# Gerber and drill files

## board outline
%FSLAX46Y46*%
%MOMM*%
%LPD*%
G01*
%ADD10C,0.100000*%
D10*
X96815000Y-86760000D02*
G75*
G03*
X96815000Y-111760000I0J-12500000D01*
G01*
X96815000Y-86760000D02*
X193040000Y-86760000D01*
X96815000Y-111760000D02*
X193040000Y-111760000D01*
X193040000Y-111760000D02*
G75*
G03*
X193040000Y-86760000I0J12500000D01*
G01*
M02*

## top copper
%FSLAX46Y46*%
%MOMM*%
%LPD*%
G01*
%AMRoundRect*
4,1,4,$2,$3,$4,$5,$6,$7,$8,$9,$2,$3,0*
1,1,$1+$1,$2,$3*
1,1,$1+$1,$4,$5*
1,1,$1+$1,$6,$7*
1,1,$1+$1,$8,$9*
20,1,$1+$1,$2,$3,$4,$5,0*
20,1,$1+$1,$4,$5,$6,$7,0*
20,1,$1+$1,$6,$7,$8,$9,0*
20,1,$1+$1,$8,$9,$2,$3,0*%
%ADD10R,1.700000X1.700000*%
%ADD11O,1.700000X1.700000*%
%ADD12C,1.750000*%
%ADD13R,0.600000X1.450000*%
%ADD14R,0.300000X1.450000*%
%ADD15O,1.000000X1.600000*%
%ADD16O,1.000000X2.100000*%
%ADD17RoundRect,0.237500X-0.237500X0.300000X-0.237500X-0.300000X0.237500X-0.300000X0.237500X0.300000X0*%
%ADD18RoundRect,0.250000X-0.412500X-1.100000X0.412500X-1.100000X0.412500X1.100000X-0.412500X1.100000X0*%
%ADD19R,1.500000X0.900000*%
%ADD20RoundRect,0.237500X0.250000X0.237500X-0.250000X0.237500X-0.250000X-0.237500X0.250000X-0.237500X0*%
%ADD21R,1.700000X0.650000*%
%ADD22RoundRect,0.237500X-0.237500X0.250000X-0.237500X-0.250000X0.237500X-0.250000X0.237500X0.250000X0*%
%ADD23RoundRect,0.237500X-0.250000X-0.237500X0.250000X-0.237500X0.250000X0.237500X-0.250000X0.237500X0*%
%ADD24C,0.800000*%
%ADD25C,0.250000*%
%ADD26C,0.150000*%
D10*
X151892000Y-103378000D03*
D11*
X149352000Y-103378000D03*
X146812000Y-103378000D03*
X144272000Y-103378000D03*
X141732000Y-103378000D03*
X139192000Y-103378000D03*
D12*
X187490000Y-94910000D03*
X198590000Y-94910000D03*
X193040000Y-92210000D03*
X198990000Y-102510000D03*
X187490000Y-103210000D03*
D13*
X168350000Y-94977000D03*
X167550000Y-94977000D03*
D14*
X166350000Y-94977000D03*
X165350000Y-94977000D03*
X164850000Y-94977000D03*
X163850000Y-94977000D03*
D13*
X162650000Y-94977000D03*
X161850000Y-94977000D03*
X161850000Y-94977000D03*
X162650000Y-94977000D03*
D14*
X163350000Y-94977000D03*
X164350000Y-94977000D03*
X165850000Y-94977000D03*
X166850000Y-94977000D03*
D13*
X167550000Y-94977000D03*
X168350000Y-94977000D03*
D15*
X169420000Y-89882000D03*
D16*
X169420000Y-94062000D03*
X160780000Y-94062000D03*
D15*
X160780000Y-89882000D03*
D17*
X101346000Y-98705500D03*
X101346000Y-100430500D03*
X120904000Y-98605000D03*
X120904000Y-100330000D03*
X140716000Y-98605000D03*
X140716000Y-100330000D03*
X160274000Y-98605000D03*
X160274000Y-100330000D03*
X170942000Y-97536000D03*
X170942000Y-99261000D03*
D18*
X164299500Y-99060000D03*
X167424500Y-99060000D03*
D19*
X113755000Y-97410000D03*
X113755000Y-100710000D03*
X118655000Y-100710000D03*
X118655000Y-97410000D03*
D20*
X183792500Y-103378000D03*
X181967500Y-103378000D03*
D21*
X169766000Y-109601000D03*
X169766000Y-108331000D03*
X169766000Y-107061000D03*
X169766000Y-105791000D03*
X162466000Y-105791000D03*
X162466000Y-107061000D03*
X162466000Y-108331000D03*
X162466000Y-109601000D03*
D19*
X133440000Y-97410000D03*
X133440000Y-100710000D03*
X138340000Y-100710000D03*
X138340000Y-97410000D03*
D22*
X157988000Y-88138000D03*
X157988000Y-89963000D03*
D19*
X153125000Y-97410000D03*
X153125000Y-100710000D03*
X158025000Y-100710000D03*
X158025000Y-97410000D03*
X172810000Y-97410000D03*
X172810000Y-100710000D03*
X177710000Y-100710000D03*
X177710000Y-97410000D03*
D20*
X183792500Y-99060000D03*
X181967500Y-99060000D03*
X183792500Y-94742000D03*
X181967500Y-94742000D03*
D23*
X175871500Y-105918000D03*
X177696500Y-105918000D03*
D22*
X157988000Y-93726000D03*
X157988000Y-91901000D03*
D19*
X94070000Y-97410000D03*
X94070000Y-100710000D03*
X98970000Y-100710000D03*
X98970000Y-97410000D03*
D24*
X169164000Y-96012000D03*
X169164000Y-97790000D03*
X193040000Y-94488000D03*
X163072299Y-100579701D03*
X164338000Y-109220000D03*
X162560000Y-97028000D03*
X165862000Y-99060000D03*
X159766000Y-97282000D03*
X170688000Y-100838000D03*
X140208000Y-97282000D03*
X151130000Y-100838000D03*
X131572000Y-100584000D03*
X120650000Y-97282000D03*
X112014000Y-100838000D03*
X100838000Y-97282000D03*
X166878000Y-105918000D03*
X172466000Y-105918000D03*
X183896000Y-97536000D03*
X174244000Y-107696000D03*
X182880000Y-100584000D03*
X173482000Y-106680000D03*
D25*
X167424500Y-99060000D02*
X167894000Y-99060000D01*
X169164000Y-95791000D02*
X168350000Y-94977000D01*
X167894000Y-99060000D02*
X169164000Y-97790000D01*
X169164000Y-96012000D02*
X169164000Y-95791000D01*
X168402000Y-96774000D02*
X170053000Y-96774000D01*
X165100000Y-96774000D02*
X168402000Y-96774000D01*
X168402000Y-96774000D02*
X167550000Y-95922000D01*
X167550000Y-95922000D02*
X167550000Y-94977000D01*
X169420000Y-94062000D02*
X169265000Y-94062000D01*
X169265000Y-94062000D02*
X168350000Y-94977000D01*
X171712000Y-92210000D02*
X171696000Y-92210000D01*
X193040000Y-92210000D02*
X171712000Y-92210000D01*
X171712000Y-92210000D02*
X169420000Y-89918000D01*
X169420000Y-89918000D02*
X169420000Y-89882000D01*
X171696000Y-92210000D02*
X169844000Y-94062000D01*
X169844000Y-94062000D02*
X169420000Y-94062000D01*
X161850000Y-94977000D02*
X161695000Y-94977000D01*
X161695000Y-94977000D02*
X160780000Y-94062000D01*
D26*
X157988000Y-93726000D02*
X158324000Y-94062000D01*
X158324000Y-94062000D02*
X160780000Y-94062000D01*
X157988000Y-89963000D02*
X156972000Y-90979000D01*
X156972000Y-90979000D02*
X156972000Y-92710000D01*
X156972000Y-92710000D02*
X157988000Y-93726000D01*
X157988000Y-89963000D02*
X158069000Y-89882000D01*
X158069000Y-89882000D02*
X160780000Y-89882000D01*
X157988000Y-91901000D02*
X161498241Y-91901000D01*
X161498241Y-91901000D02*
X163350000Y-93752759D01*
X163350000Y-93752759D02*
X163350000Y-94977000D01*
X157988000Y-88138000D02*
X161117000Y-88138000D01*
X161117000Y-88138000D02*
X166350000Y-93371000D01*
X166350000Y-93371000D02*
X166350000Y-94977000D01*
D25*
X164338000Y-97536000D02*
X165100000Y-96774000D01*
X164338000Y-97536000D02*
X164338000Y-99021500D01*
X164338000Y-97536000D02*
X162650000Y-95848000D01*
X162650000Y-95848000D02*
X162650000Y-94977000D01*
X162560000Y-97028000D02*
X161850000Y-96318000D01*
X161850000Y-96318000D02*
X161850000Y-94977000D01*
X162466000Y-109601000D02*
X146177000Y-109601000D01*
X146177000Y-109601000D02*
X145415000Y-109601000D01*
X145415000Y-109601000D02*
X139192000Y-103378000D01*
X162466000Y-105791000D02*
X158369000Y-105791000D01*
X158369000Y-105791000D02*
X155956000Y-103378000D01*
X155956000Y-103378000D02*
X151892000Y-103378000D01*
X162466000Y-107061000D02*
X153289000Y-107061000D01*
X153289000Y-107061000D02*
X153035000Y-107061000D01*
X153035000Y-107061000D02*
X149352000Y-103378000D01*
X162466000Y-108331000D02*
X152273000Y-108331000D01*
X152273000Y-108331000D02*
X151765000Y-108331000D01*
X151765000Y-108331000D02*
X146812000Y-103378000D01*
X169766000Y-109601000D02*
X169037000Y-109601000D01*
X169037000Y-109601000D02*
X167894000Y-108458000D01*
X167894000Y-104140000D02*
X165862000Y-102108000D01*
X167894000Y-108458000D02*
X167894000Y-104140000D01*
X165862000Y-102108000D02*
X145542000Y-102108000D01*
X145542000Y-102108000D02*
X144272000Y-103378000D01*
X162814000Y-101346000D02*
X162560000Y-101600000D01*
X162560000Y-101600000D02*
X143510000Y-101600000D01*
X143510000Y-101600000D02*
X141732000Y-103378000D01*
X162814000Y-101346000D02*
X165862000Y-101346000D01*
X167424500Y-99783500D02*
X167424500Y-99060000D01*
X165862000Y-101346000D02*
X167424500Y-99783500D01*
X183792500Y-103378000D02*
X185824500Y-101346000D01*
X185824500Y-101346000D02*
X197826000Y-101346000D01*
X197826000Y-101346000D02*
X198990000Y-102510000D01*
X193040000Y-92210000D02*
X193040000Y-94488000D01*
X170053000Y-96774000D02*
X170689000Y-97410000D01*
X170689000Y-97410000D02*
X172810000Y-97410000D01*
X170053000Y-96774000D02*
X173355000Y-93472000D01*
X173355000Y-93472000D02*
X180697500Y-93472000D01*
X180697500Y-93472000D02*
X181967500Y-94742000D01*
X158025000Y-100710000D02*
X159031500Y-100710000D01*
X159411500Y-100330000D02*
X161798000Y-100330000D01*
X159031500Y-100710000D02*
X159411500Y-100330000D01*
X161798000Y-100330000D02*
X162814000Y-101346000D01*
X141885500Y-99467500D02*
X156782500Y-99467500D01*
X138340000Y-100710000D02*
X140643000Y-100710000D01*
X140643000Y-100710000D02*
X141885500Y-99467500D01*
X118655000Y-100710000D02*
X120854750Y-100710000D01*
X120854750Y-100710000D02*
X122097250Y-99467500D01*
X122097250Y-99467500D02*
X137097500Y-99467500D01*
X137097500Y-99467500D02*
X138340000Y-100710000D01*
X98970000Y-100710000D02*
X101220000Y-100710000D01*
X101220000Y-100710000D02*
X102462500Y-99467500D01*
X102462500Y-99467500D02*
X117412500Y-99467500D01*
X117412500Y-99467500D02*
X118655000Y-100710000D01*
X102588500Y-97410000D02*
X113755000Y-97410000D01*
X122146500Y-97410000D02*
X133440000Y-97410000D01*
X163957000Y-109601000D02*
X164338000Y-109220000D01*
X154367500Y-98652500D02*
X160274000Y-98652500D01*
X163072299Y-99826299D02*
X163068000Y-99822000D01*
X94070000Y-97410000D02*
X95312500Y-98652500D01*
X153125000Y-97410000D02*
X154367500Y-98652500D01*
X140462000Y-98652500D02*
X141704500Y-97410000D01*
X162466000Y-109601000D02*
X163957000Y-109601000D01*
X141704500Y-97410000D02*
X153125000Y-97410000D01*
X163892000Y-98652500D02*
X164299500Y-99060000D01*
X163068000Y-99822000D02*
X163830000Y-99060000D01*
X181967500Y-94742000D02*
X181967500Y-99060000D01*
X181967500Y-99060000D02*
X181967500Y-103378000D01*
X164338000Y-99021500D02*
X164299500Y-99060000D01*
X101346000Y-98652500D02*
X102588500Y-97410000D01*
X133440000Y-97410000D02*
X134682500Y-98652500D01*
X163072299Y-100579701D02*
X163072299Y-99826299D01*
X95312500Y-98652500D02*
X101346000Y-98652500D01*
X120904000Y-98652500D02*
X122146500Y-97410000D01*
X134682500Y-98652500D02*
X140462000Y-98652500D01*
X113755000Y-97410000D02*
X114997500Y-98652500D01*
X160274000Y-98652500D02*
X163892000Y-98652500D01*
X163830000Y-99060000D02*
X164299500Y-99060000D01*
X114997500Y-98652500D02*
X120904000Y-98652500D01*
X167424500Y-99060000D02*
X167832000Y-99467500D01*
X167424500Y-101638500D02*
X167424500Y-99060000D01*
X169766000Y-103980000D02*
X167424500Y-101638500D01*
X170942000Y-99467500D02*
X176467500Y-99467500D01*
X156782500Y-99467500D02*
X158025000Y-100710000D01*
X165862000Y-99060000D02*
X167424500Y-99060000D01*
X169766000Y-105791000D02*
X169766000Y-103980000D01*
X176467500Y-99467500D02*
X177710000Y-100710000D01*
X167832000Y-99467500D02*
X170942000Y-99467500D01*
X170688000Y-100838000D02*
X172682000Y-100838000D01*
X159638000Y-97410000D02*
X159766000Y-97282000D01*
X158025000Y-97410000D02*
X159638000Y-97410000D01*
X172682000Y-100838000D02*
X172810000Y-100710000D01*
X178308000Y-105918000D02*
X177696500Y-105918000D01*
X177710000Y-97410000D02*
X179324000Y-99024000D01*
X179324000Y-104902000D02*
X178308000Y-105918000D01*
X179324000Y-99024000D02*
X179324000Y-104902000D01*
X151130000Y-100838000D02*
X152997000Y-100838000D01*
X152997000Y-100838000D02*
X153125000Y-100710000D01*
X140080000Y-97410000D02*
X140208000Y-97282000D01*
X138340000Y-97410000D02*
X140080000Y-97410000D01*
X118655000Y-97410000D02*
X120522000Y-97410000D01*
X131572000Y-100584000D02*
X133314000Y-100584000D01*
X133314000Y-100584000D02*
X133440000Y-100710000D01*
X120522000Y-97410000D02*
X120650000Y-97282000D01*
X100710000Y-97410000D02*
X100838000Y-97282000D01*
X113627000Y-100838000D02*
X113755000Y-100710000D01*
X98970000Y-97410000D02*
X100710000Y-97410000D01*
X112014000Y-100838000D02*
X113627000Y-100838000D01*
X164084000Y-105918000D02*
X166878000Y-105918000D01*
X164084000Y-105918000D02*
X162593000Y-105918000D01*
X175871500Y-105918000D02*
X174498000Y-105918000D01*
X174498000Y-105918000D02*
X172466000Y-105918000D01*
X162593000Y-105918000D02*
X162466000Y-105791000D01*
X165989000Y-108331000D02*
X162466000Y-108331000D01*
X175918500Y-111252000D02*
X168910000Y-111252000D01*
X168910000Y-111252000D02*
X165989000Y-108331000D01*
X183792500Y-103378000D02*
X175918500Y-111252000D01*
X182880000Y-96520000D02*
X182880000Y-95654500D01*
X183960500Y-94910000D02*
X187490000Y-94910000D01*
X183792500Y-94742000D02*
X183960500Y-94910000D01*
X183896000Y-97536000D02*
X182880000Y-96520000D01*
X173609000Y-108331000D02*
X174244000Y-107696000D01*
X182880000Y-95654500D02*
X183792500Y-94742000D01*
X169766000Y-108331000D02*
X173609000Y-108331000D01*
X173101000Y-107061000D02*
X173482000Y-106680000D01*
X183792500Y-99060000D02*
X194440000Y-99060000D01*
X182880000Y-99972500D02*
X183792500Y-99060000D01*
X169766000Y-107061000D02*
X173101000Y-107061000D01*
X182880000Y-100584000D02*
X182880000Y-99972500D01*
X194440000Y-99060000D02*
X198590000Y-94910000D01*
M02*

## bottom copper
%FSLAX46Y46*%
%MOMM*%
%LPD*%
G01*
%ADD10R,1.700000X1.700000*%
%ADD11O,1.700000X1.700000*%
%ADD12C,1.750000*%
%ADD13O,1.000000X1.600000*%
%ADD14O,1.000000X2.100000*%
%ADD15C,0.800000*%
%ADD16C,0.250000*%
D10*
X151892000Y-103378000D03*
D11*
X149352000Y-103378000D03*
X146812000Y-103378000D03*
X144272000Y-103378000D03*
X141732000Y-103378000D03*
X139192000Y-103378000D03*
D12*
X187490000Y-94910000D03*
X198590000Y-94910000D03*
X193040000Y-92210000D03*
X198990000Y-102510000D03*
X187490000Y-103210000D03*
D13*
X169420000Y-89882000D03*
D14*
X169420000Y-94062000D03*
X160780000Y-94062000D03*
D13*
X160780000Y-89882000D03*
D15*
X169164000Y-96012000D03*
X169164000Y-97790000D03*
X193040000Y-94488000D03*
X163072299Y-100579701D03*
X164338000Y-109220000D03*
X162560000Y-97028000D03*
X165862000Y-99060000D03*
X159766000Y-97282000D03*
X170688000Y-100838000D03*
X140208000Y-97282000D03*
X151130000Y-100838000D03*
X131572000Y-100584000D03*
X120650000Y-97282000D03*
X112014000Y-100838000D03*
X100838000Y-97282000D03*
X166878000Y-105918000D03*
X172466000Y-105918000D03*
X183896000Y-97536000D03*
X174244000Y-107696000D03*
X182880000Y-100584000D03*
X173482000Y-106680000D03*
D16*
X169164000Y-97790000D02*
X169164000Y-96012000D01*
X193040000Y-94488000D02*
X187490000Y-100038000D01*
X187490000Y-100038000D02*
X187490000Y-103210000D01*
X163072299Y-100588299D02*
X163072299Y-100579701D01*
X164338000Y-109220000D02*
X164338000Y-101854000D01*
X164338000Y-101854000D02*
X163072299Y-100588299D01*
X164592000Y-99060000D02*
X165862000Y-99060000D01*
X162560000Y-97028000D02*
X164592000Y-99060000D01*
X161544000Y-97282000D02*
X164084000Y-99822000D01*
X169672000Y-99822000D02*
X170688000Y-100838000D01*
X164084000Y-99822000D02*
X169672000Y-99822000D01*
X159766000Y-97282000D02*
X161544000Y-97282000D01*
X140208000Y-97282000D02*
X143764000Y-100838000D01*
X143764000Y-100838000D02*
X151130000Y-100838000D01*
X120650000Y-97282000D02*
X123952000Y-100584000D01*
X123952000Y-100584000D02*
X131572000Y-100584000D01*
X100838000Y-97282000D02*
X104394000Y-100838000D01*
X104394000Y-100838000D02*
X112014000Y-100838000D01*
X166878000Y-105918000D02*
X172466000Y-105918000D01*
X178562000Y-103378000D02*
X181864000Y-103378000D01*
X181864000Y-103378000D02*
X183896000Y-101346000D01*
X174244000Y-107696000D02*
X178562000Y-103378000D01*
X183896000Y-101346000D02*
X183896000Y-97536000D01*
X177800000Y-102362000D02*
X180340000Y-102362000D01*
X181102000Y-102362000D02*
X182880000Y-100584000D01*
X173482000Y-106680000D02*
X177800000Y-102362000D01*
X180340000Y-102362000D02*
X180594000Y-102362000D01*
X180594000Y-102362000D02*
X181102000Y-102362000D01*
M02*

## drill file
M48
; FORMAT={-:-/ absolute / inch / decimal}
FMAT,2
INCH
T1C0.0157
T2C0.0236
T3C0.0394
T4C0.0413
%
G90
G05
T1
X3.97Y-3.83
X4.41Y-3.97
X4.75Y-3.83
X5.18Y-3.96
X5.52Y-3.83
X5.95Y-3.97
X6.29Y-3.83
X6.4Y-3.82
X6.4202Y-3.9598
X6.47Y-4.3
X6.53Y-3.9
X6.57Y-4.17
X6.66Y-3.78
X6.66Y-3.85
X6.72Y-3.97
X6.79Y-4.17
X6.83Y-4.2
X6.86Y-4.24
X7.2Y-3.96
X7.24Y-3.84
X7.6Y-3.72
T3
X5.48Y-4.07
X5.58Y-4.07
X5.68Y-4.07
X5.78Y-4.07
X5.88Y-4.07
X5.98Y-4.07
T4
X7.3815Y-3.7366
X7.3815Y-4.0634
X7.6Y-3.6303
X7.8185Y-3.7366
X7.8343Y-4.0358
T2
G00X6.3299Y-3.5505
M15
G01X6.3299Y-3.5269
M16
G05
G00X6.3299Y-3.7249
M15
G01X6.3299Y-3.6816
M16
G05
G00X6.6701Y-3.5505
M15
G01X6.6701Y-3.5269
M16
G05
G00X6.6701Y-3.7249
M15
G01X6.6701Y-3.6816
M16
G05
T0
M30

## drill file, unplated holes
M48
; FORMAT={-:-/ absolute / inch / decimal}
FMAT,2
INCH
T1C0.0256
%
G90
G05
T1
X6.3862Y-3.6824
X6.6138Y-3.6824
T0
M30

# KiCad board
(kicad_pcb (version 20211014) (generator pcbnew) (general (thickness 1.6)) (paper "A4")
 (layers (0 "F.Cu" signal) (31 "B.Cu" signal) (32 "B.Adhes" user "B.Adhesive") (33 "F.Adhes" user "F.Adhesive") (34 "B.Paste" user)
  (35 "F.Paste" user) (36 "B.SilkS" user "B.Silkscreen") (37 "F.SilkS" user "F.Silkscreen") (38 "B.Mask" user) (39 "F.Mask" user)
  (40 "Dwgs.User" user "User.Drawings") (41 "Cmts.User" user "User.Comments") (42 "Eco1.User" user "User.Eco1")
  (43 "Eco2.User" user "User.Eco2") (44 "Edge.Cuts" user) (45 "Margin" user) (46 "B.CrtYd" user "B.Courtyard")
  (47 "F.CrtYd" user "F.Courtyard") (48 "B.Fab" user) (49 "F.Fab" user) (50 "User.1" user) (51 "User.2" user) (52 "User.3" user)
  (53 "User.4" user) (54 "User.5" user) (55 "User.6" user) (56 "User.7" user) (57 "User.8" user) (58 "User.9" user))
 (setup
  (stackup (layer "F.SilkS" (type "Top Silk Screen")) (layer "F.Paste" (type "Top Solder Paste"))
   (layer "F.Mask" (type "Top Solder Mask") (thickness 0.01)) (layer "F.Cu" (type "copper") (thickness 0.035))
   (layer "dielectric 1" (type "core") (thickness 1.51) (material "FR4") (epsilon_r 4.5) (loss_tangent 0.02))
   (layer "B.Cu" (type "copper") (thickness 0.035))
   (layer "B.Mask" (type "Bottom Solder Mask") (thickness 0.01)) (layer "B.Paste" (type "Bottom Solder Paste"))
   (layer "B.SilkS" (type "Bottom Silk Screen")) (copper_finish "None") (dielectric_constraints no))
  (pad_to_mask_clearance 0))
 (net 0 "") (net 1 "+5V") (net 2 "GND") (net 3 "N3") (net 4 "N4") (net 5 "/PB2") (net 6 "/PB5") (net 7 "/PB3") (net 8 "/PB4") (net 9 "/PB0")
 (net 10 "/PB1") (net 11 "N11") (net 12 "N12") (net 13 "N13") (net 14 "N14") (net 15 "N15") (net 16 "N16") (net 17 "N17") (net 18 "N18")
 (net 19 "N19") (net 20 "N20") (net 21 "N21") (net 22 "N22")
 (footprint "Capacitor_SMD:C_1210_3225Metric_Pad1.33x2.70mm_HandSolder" (layer "F.Cu") (at 165.862 99.06)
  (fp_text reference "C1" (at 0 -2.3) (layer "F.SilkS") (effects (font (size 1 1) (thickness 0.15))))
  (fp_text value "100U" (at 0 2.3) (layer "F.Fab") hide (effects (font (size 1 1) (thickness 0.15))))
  (pad "1" smd roundrect (at -1.5625 0) (size 1.325 2.7) (layers "F.Cu" "F.Paste" "F.Mask") (roundrect_rratio 0.1886792453) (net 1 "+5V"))
  (pad "2" smd roundrect (at 1.5625 0) (size 1.325 2.7) (layers "F.Cu" "F.Paste" "F.Mask") (roundrect_rratio 0.1886792453) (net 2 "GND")))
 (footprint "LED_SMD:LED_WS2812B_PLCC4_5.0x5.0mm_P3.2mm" (layer "F.Cu") (at 116.205 99.06)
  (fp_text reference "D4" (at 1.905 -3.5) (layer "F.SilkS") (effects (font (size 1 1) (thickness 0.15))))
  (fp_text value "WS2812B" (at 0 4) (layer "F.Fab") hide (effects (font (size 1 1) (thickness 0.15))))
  (pad "1" smd rect (at -2.45 -1.65) (size 1.5 0.9) (layers "F.Cu" "F.Paste" "F.Mask") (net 1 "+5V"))
  (pad "2" smd rect (at -2.45 1.65) (size 1.5 0.9) (layers "F.Cu" "F.Paste" "F.Mask") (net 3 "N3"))
  (pad "3" smd rect (at 2.45 1.65) (size 1.5 0.9) (layers "F.Cu" "F.Paste" "F.Mask") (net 2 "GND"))
  (pad "4" smd rect (at 2.45 -1.65) (size 1.5 0.9) (layers "F.Cu" "F.Paste" "F.Mask") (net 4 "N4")))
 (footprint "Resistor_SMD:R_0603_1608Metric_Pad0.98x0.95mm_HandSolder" (layer "F.Cu") (at 182.88 103.378 180)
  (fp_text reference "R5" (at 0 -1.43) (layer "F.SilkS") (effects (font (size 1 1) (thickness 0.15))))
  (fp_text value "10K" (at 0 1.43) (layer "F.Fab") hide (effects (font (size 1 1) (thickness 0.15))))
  (pad "1" smd roundrect (at -0.9125 0 180) (size 0.975 0.95) (layers "F.Cu" "F.Paste" "F.Mask") (roundrect_rratio 0.25) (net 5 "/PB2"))
  (pad "2" smd roundrect (at 0.9125 0 180) (size 0.975 0.95) (layers "F.Cu" "F.Paste" "F.Mask") (roundrect_rratio 0.25) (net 1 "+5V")))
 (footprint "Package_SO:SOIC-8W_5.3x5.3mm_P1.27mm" (layer "F.Cu") (at 166.116 107.696 180)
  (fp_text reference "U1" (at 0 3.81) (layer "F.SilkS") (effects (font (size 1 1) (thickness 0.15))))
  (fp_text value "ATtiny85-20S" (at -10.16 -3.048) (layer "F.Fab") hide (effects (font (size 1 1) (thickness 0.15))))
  (pad "1" smd rect (at -3.65 -1.905 180) (size 1.7 0.65) (layers "F.Cu" "F.Paste" "F.Mask") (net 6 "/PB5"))
  (pad "2" smd rect (at -3.65 -0.635 180) (size 1.7 0.65) (layers "F.Cu" "F.Paste" "F.Mask") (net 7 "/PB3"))
  (pad "3" smd rect (at -3.65 0.635 180) (size 1.7 0.65) (layers "F.Cu" "F.Paste" "F.Mask") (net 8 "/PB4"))
  (pad "4" smd rect (at -3.65 1.905 180) (size 1.7 0.65) (layers "F.Cu" "F.Paste" "F.Mask") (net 2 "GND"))
  (pad "5" smd rect (at 3.65 1.905 180) (size 1.7 0.65) (layers "F.Cu" "F.Paste" "F.Mask") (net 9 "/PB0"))
  (pad "6" smd rect (at 3.65 0.635 180) (size 1.7 0.65) (layers "F.Cu" "F.Paste" "F.Mask") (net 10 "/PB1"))
  (pad "7" smd rect (at 3.65 -0.635 180) (size 1.7 0.65) (layers "F.Cu" "F.Paste" "F.Mask") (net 5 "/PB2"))
  (pad "8" smd rect (at 3.65 -1.905 180) (size 1.7 0.65) (layers "F.Cu" "F.Paste" "F.Mask") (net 1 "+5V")))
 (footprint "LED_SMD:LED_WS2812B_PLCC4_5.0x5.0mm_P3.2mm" (layer "F.Cu") (at 135.89 99.06)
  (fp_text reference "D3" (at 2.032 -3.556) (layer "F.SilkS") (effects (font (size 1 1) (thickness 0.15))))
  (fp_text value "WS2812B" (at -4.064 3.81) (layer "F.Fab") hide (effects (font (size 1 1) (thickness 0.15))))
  (pad "1" smd rect (at -2.45 -1.65) (size 1.5 0.9) (layers "F.Cu" "F.Paste" "F.Mask") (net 1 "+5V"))
  (pad "2" smd rect (at -2.45 1.65) (size 1.5 0.9) (layers "F.Cu" "F.Paste" "F.Mask") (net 4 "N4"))
  (pad "3" smd rect (at 2.45 1.65) (size 1.5 0.9) (layers "F.Cu" "F.Paste" "F.Mask") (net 2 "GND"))
  (pad "4" smd rect (at 2.45 -1.65) (size 1.5 0.9) (layers "F.Cu" "F.Paste" "F.Mask") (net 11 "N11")))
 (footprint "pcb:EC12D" (layer "F.Cu") (at 193.04 99.06)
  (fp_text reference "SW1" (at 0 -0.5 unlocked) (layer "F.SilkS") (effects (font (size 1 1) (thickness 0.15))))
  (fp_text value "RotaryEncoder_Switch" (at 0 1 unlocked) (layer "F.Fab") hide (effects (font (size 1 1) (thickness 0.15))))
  (pad "A" thru_hole circle (at -5.55 -4.15) (size 1.75 1.75) (drill 1.05) (layers *.Cu *.Mask) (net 7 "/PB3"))
  (pad "B" thru_hole circle (at 5.55 -4.15) (size 1.75 1.75) (drill 1.05) (layers *.Cu *.Mask) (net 8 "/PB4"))
  (pad "C" thru_hole circle (at 0 -6.85) (size 1.75 1.75) (drill 1.05) (layers *.Cu *.Mask) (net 2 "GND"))
  (pad "S1" thru_hole circle (at 5.95 3.45) (size 1.75 1.75) (drill 1.05) (layers *.Cu *.Mask) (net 5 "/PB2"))
  (pad "S2" thru_hole circle (at -5.55 4.15) (size 1.75 1.75) (drill 1.05) (layers *.Cu *.Mask) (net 2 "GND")))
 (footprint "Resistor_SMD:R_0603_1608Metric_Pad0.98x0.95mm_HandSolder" (layer "F.Cu") (at 157.988 89.0505 -90)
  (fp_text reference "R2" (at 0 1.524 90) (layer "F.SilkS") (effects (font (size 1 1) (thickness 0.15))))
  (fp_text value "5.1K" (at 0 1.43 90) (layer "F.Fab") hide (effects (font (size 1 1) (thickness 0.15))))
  (pad "1" smd roundrect (at -0.9125 0 270) (size 0.975 0.95) (layers "F.Cu" "F.Paste" "F.Mask") (roundrect_rratio 0.25) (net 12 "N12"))
  (pad "2" smd roundrect (at 0.9125 0 270) (size 0.975 0.95) (layers "F.Cu" "F.Paste" "F.Mask") (roundrect_rratio 0.25) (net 2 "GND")))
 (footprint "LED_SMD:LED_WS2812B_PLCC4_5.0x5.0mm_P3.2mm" (layer "F.Cu") (at 155.575 99.06)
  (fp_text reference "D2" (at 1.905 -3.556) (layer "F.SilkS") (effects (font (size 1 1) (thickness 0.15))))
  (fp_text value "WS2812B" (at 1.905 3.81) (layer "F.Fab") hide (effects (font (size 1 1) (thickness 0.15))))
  (pad "1" smd rect (at -2.45 -1.65) (size 1.5 0.9) (layers "F.Cu" "F.Paste" "F.Mask") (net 1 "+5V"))
  (pad "2" smd rect (at -2.45 1.65) (size 1.5 0.9) (layers "F.Cu" "F.Paste" "F.Mask") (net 11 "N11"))
  (pad "3" smd rect (at 2.45 1.65) (size 1.5 0.9) (layers "F.Cu" "F.Paste" "F.Mask") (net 2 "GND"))
  (pad "4" smd rect (at 2.45 -1.65) (size 1.5 0.9) (layers "F.Cu" "F.Paste" "F.Mask") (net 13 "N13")))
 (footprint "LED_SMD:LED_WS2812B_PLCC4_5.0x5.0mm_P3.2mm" (layer "F.Cu") (at 175.26 99.06)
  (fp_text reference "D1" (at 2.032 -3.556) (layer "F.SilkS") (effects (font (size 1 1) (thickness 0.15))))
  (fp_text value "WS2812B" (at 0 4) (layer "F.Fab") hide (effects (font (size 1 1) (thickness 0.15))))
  (pad "1" smd rect (at -2.45 -1.65) (size 1.5 0.9) (layers "F.Cu" "F.Paste" "F.Mask") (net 1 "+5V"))
  (pad "2" smd rect (at -2.45 1.65) (size 1.5 0.9) (layers "F.Cu" "F.Paste" "F.Mask") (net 13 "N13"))
  (pad "3" smd rect (at 2.45 1.65) (size 1.5 0.9) (layers "F.Cu" "F.Paste" "F.Mask") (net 2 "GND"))
  (pad "4" smd rect (at 2.45 -1.65) (size 1.5 0.9) (layers "F.Cu" "F.Paste" "F.Mask") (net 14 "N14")))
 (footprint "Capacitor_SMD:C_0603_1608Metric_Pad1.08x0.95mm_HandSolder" (layer "F.Cu") (at 170.942 98.3985 -90)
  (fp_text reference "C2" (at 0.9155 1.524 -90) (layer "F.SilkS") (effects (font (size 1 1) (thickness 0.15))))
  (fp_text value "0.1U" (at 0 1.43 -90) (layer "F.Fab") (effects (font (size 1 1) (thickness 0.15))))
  (pad "1" smd roundrect (at -0.8625 0 270) (size 1.075 0.95) (layers "F.Cu" "F.Paste" "F.Mask") (roundrect_rratio 0.25) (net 1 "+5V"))
  (pad "2" smd roundrect (at 0.8625 0 270) (size 1.075 0.95) (layers "F.Cu" "F.Paste" "F.Mask") (roundrect_rratio 0.25) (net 2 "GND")))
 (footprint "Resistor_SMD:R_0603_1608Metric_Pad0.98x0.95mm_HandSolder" (layer "F.Cu") (at 182.88 99.06 180)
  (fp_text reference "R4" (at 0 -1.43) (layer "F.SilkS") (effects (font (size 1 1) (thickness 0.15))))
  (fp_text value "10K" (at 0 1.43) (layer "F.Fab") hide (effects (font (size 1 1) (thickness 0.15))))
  (pad "1" smd roundrect (at -0.9125 0 180) (size 0.975 0.95) (layers "F.Cu" "F.Paste" "F.Mask") (roundrect_rratio 0.25) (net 8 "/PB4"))
  (pad "2" smd roundrect (at 0.9125 0 180) (size 0.975 0.95) (layers "F.Cu" "F.Paste" "F.Mask") (roundrect_rratio 0.25) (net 1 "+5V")))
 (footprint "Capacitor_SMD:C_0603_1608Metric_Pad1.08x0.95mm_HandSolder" (layer "F.Cu") (at 140.716 99.4675 -90)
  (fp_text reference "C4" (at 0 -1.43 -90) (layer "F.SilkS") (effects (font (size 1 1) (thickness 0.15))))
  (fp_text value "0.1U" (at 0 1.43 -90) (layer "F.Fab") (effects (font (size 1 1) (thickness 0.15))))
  (pad "1" smd roundrect (at -0.8625 0 270) (size 1.075 0.95) (layers "F.Cu" "F.Paste" "F.Mask") (roundrect_rratio 0.25) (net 1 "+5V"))
  (pad "2" smd roundrect (at 0.8625 0 270) (size 1.075 0.95) (layers "F.Cu" "F.Paste" "F.Mask") (roundrect_rratio 0.25) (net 2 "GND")))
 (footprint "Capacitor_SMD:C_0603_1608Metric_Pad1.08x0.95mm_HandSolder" (layer "F.Cu") (at 160.274 99.4675 -90)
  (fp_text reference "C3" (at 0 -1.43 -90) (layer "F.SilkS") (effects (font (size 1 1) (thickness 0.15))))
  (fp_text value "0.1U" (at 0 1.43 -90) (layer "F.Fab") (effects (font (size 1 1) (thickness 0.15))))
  (pad "1" smd roundrect (at -0.8625 0 270) (size 1.075 0.95) (layers "F.Cu" "F.Paste" "F.Mask") (roundrect_rratio 0.25) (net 1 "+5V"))
  (pad "2" smd roundrect (at 0.8625 0 270) (size 1.075 0.95) (layers "F.Cu" "F.Paste" "F.Mask") (roundrect_rratio 0.25) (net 2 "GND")))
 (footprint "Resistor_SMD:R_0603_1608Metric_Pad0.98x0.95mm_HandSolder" (layer "F.Cu") (at 182.88 94.742 180)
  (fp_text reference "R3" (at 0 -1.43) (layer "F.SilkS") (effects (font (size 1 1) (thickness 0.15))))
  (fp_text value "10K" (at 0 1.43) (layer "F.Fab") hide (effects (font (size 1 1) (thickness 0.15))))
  (pad "1" smd roundrect (at -0.9125 0 180) (size 0.975 0.95) (layers "F.Cu" "F.Paste" "F.Mask") (roundrect_rratio 0.25) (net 7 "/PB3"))
  (pad "2" smd roundrect (at 0.9125 0 180) (size 0.975 0.95) (layers "F.Cu" "F.Paste" "F.Mask") (roundrect_rratio 0.25) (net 1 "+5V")))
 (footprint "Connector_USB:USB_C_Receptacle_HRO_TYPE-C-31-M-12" (layer "F.Cu") (at 165.1 90.932 180)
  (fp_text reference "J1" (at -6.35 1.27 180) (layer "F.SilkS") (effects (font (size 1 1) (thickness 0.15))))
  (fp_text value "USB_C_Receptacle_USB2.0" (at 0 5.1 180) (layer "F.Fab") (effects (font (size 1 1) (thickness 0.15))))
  (pad "" np_thru_hole circle (at 2.89 -2.6 180) (size 0.65 0.65) (drill 0.65) (layers *.Cu *.Mask))
  (pad "" np_thru_hole circle (at -2.89 -2.6 180) (size 0.65 0.65) (drill 0.65) (layers *.Cu *.Mask))
  (pad "A1" smd rect (at -3.25 -4.045 180) (size 0.6 1.45) (layers "F.Cu" "F.Paste" "F.Mask") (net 2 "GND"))
  (pad "A4" smd rect (at -2.45 -4.045 180) (size 0.6 1.45) (layers "F.Cu" "F.Paste" "F.Mask") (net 1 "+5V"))
  (pad "A5" smd rect (at -1.25 -4.045 180) (size 0.3 1.45) (layers "F.Cu" "F.Paste" "F.Mask") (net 12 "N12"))
  (pad "A6" smd rect (at -0.25 -4.045 180) (size 0.3 1.45) (layers "F.Cu" "F.Paste" "F.Mask") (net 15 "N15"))
  (pad "A7" smd rect (at 0.25 -4.045 180) (size 0.3 1.45) (layers "F.Cu" "F.Paste" "F.Mask") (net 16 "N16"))
  (pad "A8" smd rect (at 1.25 -4.045 180) (size 0.3 1.45) (layers "F.Cu" "F.Paste" "F.Mask") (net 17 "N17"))
  (pad "A9" smd rect (at 2.45 -4.045 180) (size 0.6 1.45) (layers "F.Cu" "F.Paste" "F.Mask") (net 1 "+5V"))
  (pad "A12" smd rect (at 3.25 -4.045 180) (size 0.6 1.45) (layers "F.Cu" "F.Paste" "F.Mask") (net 2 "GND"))
  (pad "B1" smd rect (at 3.25 -4.045 180) (size 0.6 1.45) (layers "F.Cu" "F.Paste" "F.Mask") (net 2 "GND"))
  (pad "B4" smd rect (at 2.45 -4.045 180) (size 0.6 1.45) (layers "F.Cu" "F.Paste" "F.Mask") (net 1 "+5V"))
  (pad "B5" smd rect (at 1.75 -4.045 180) (size 0.3 1.45) (layers "F.Cu" "F.Paste" "F.Mask") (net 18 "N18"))
  (pad "B6" smd rect (at 0.75 -4.045 180) (size 0.3 1.45) (layers "F.Cu" "F.Paste" "F.Mask") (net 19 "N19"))
  (pad "B7" smd rect (at -0.75 -4.045 180) (size 0.3 1.45) (layers "F.Cu" "F.Paste" "F.Mask") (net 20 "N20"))
  (pad "B8" smd rect (at -1.75 -4.045 180) (size 0.3 1.45) (layers "F.Cu" "F.Paste" "F.Mask") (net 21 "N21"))
  (pad "B9" smd rect (at -2.45 -4.045 180) (size 0.6 1.45) (layers "F.Cu" "F.Paste" "F.Mask") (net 1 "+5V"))
  (pad "B12" smd rect (at -3.25 -4.045 180) (size 0.6 1.45) (layers "F.Cu" "F.Paste" "F.Mask") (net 2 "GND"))
  (pad "S1" thru_hole oval (at -4.32 1.05 180) (size 1 1.6) (drill oval 0.6 1.2) (layers *.Cu *.Mask) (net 2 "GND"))
  (pad "S1" thru_hole oval (at -4.32 -3.13 180) (size 1 2.1) (drill oval 0.6 1.7) (layers *.Cu *.Mask) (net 2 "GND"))
  (pad "S1" thru_hole oval (at 4.32 1.05 180) (size 1 1.6) (drill oval 0.6 1.2) (layers *.Cu *.Mask) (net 2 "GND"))
  (pad "S1" thru_hole oval (at 4.32 -3.13 180) (size 1 2.1) (drill oval 0.6 1.7) (layers *.Cu *.Mask) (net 2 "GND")))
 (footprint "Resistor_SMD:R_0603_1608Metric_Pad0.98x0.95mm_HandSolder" (layer "F.Cu") (at 176.784 105.918)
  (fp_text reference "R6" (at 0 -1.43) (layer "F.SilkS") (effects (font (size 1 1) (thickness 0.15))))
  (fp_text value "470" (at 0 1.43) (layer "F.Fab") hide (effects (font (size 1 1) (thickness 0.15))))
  (pad "1" smd roundrect (at -0.9125 0) (size 0.975 0.95) (layers "F.Cu" "F.Paste" "F.Mask") (roundrect_rratio 0.25) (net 9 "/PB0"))
  (pad "2" smd roundrect (at 0.9125 0) (size 0.975 0.95) (layers "F.Cu" "F.Paste" "F.Mask") (roundrect_rratio 0.25) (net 14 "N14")))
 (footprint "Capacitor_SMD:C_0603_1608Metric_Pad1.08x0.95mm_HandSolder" (layer "F.Cu") (at 120.904 99.4675 -90)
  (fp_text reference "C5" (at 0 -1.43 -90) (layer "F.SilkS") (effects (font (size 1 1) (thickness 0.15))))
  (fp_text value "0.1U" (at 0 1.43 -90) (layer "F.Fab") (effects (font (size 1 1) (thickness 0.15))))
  (pad "1" smd roundrect (at -0.8625 0 270) (size 1.075 0.95) (layers "F.Cu" "F.Paste" "F.Mask") (roundrect_rratio 0.25) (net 1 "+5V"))
  (pad "2" smd roundrect (at 0.8625 0 270) (size 1.075 0.95) (layers "F.Cu" "F.Paste" "F.Mask") (roundrect_rratio 0.25) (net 2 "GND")))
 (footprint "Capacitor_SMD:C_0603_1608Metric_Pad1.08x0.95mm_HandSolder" (layer "F.Cu") (at 101.346 99.568 -90)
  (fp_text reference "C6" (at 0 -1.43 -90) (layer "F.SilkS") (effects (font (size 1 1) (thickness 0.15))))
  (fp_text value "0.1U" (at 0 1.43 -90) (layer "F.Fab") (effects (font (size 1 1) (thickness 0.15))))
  (pad "1" smd roundrect (at -0.8625 0 270) (size 1.075 0.95) (layers "F.Cu" "F.Paste" "F.Mask") (roundrect_rratio 0.25) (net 1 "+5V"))
  (pad "2" smd roundrect (at 0.8625 0 270) (size 1.075 0.95) (layers "F.Cu" "F.Paste" "F.Mask") (roundrect_rratio 0.25) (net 2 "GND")))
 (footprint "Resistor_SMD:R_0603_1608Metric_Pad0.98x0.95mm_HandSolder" (layer "F.Cu") (at 157.988 92.8135 -90)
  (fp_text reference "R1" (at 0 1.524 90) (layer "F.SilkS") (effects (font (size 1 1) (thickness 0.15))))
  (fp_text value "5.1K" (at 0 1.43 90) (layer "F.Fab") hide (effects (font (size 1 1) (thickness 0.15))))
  (pad "1" smd roundrect (at -0.9125 0 270) (size 0.975 0.95) (layers "F.Cu" "F.Paste" "F.Mask") (roundrect_rratio 0.25) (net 18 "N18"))
  (pad "2" smd roundrect (at 0.9125 0 270) (size 0.975 0.95) (layers "F.Cu" "F.Paste" "F.Mask") (roundrect_rratio 0.25) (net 2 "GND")))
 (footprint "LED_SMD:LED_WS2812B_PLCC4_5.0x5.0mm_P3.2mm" (layer "F.Cu") (at 96.52 99.06)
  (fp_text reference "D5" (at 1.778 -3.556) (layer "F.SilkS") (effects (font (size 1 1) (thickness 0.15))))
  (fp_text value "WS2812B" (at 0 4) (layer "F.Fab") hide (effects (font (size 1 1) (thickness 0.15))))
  (pad "1" smd rect (at -2.45 -1.65) (size 1.5 0.9) (layers "F.Cu" "F.Paste" "F.Mask") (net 1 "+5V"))
  (pad "2" smd rect (at -2.45 1.65) (size 1.5 0.9) (layers "F.Cu" "F.Paste" "F.Mask") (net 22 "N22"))
  (pad "3" smd rect (at 2.45 1.65) (size 1.5 0.9) (layers "F.Cu" "F.Paste" "F.Mask") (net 2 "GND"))
  (pad "4" smd rect (at 2.45 -1.65) (size 1.5 0.9) (layers "F.Cu" "F.Paste" "F.Mask") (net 3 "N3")))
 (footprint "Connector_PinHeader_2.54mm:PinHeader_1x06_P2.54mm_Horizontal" (layer "F.Cu") (at 151.892 103.378 -90)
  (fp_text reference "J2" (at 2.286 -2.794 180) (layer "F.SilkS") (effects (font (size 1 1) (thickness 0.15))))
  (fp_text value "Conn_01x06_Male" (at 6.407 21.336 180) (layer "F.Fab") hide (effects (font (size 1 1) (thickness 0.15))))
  (pad "1" thru_hole rect (at 0 0 270) (size 1.7 1.7) (drill 1) (layers *.Cu *.Mask) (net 9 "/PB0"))
  (pad "2" thru_hole oval (at 0 2.54 270) (size 1.7 1.7) (drill 1) (layers *.Cu *.Mask) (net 10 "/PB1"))
  (pad "3" thru_hole oval (at 0 5.08 270) (size 1.7 1.7) (drill 1) (layers *.Cu *.Mask) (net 5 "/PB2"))
  (pad "4" thru_hole oval (at 0 7.62 270) (size 1.7 1.7) (drill 1) (layers *.Cu *.Mask) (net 6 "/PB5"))
  (pad "5" thru_hole oval (at 0 10.16 270) (size 1.7 1.7) (drill 1) (layers *.Cu *.Mask) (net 2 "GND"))
  (pad "6" thru_hole oval (at 0 12.7 270) (size 1.7 1.7) (drill 1) (layers *.Cu *.Mask) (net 1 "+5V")))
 (gr_arc (start 96.815 111.76) (mid 84.315 99.26) (end 96.815 86.76) (layer "Edge.Cuts") (width 0.1))
 (gr_line (start 96.815 86.76) (end 193.04 86.76) (layer "Edge.Cuts") (width 0.1))
 (gr_line (start 96.815 111.76) (end 193.04 111.76) (layer "Edge.Cuts") (width 0.1))
 (gr_arc (start 193.04 86.76) (mid 205.54 99.26) (end 193.04 111.76) (layer "Edge.Cuts") (width 0.1))
 (segment (start 102.5885 97.41) (end 113.755 97.41) (width 0.25) (layer "F.Cu") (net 1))
 (segment (start 122.1465 97.41) (end 133.44 97.41) (width 0.25) (layer "F.Cu") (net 1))
 (segment (start 163.957 109.601) (end 164.338 109.22) (width 0.25) (layer "F.Cu") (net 1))
 (segment (start 146.177 109.601) (end 145.415 109.601) (width 0.25) (layer "F.Cu") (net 1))
 (segment (start 154.3675 98.6525) (end 160.274 98.6525) (width 0.25) (layer "F.Cu") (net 1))
 (segment (start 163.072299 99.826299) (end 163.068 99.822) (width 0.25) (layer "F.Cu") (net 1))
 (segment (start 94.07 97.41) (end 95.3125 98.6525) (width 0.25) (layer "F.Cu") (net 1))
 (segment (start 153.125 97.41) (end 154.3675 98.6525) (width 0.25) (layer "F.Cu") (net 1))
 (segment (start 173.355 93.472) (end 180.6975 93.472) (width 0.25) (layer "F.Cu") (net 1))
 (segment (start 140.462 98.6525) (end 141.7045 97.41) (width 0.25) (layer "F.Cu") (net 1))
 (segment (start 170.053 96.774) (end 170.689 97.41) (width 0.25) (layer "F.Cu") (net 1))
 (segment (start 164.338 97.536) (end 164.338 99.0215) (width 0.25) (layer "F.Cu") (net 1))
 (segment (start 162.466 109.601) (end 163.957 109.601) (width 0.25) (layer "F.Cu") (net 1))
 (segment (start 164.338 97.536) (end 162.65 95.848) (width 0.25) (layer "F.Cu") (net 1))
 (segment (start 141.7045 97.41) (end 153.125 97.41) (width 0.25) (layer "F.Cu") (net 1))
 (segment (start 170.689 97.41) (end 172.81 97.41) (width 0.25) (layer "F.Cu") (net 1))
 (segment (start 163.892 98.6525) (end 164.2995 99.06) (width 0.25) (layer "F.Cu") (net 1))
 (segment (start 165.1 96.774) (end 168.402 96.774) (width 0.25) (layer "F.Cu") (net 1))
 (segment (start 163.068 99.822) (end 163.83 99.06) (width 0.25) (layer "F.Cu") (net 1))
 (segment (start 181.9675 94.742) (end 181.9675 99.06) (width 0.25) (layer "F.Cu") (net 1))
 (segment (start 181.9675 99.06) (end 181.9675 103.378) (width 0.25) (layer "F.Cu") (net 1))
 (segment (start 164.338 99.0215) (end 164.2995 99.06) (width 0.25) (layer "F.Cu") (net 1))
 (segment (start 170.053 96.774) (end 173.355 93.472) (width 0.25) (layer "F.Cu") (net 1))
 (segment (start 162.466 109.601) (end 146.177 109.601) (width 0.25) (layer "F.Cu") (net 1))
 (segment (start 101.346 98.6525) (end 102.5885 97.41) (width 0.25) (layer "F.Cu") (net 1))
 (segment (start 167.55 95.922) (end 167.55 94.977) (width 0.25) (layer "F.Cu") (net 1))
 (segment (start 168.402 96.774) (end 167.55 95.922) (width 0.25) (layer "F.Cu") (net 1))
 (segment (start 133.44 97.41) (end 134.6825 98.6525) (width 0.25) (layer "F.Cu") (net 1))
 (segment (start 164.338 97.536) (end 165.1 96.774) (width 0.25) (layer "F.Cu") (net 1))
 (segment (start 163.072299 100.579701) (end 163.072299 99.826299) (width 0.25) (layer "F.Cu") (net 1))
 (segment (start 180.6975 93.472) (end 181.9675 94.742) (width 0.25) (layer "F.Cu") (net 1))
 (segment (start 95.3125 98.6525) (end 101.346 98.6525) (width 0.25) (layer "F.Cu") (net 1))
 (segment (start 120.904 98.6525) (end 122.1465 97.41) (width 0.25) (layer "F.Cu") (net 1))
 (segment (start 134.6825 98.6525) (end 140.462 98.6525) (width 0.25) (layer "F.Cu") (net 1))
 (segment (start 113.755 97.41) (end 114.9975 98.6525) (width 0.25) (layer "F.Cu") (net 1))
 (segment (start 168.402 96.774) (end 170.053 96.774) (width 0.25) (layer "F.Cu") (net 1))
 (segment (start 160.274 98.6525) (end 163.892 98.6525) (width 0.25) (layer "F.Cu") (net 1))
 (segment (start 163.83 99.06) (end 164.2995 99.06) (width 0.25) (layer "F.Cu") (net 1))
 (segment (start 145.415 109.601) (end 139.192 103.378) (width 0.25) (layer "F.Cu") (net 1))
 (segment (start 162.65 95.848) (end 162.65 94.977) (width 0.25) (layer "F.Cu") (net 1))
 (segment (start 114.9975 98.6525) (end 120.904 98.6525) (width 0.25) (layer "F.Cu") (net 1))
 (via (at 163.072299 100.579701) (size 0.8) (drill 0.4) (layers "F.Cu" "B.Cu") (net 1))
 (via (at 164.338 109.22) (size 0.8) (drill 0.4) (layers "F.Cu" "B.Cu") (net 1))
 (segment (start 163.072299 100.588299) (end 163.072299 100.579701) (width 0.25) (layer "B.Cu") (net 1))
 (segment (start 164.338 109.22) (end 164.338 101.854) (width 0.25) (layer "B.Cu") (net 1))
 (segment (start 164.338 101.854) (end 163.072299 100.588299) (width 0.25) (layer "B.Cu") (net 1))
 (segment (start 138.34 100.71) (end 140.643 100.71) (width 0.25) (layer "F.Cu") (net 2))
 (segment (start 101.22 100.71) (end 102.4625 99.4675) (width 0.25) (layer "F.Cu") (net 2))
 (segment (start 162.814 101.346) (end 165.862 101.346) (width 0.25) (layer "F.Cu") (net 2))
 (segment (start 141.8855 99.4675) (end 156.7825 99.4675) (width 0.25) (layer "F.Cu") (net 2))
 (segment (start 158.324 94.062) (end 160.78 94.062) (width 0.15) (layer "F.Cu") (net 2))
 (segment (start 161.798 100.33) (end 162.814 101.346) (width 0.25) (layer "F.Cu") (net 2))
 (segment (start 161.85 96.318) (end 161.85 94.977) (width 0.25) (layer "F.Cu") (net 2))
 (segment (start 171.712 92.21) (end 171.696 92.21) (width 0.25) (layer "F.Cu") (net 2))
 (segment (start 167.4245 99.06) (end 167.832 99.4675) (width 0.25) (layer "F.Cu") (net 2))
 (segment (start 156.972 90.979) (end 156.972 92.71) (width 0.15) (layer "F.Cu") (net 2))
 (segment (start 157.988 89.963) (end 156.972 90.979) (width 0.15) (layer "F.Cu") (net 2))
 (segment (start 169.164 95.791) (end 168.35 94.977) (width 0.25) (layer "F.Cu") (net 2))
 (segment (start 122.09725 99.4675) (end 137.0975 99.4675) (width 0.25) (layer "F.Cu") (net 2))
 (segment (start 167.4245 99.7835) (end 167.4245 99.06) (width 0.25) (layer "F.Cu") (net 2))
 (segment (start 193.04 92.21) (end 171.712 92.21) (width 0.25) (layer "F.Cu") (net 2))
 (segment (start 167.4245 101.6385) (end 167.4245 99.06) (width 0.25) (layer "F.Cu") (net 2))
 (segment (start 143.51 101.6) (end 141.732 103.378) (width 0.25) (layer "F.Cu") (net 2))
 (segment (start 159.4115 100.33) (end 161.798 100.33) (width 0.25) (layer "F.Cu") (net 2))
 (segment (start 158.069 89.882) (end 160.78 89.882) (width 0.15) (layer "F.Cu") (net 2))
 (segment (start 165.862 101.346) (end 167.4245 99.7835) (width 0.25) (layer "F.Cu") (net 2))
 (segment (start 161.695 94.977) (end 160.78 94.062) (width 0.25) (layer "F.Cu") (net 2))
 (segment (start 169.766 103.98) (end 167.4245 101.6385) (width 0.25) (layer "F.Cu") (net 2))
 (segment (start 157.988 93.726) (end 158.324 94.062) (width 0.15) (layer "F.Cu") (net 2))
 (segment (start 169.844 94.062) (end 169.42 94.062) (width 0.25) (layer "F.Cu") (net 2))
 (segment (start 170.942 99.4675) (end 176.4675 99.4675) (width 0.25) (layer "F.Cu") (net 2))
 (segment (start 120.85475 100.71) (end 122.09725 99.4675) (width 0.25) (layer "F.Cu") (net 2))
 (segment (start 161.85 94.977) (end 161.695 94.977) (width 0.25) (layer "F.Cu") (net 2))
 (segment (start 193.04 92.21) (end 193.04 94.488) (width 0.25) (layer "F.Cu") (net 2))
 (segment (start 137.0975 99.4675) (end 138.34 100.71) (width 0.25) (layer "F.Cu") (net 2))
 (segment (start 156.7825 99.4675) (end 158.025 100.71) (width 0.25) (layer "F.Cu") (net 2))
 (segment (start 171.696 92.21) (end 169.844 94.062) (width 0.25) (layer "F.Cu") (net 2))
 (segment (start 158.025 100.71) (end 159.0315 100.71) (width 0.25) (layer "F.Cu") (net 2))
 (segment (start 118.655 100.71) (end 120.85475 100.71) (width 0.25) (layer "F.Cu") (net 2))
 (segment (start 165.862 99.06) (end 167.4245 99.06) (width 0.25) (layer "F.Cu") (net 2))
 (segment (start 162.814 101.346) (end 162.56 101.6) (width 0.25) (layer "F.Cu") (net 2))
 (segment (start 117.4125 99.4675) (end 118.655 100.71) (width 0.25) (layer "F.Cu") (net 2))
 (segment (start 162.56 97.028) (end 161.85 96.318) (width 0.25) (layer "F.Cu") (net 2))
 (segment (start 167.4245 99.06) (end 167.894 99.06) (width 0.25) (layer "F.Cu") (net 2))
 (segment (start 98.97 100.71) (end 101.22 100.71) (width 0.25) (layer "F.Cu") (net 2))
 (segment (start 169.42 94.062) (end 169.265 94.062) (width 0.25) (layer "F.Cu") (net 2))
 (segment (start 171.712 92.21) (end 169.42 89.918) (width 0.25) (layer "F.Cu") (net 2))
 (segment (start 169.766 105.791) (end 169.766 103.98) (width 0.25) (layer "F.Cu") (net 2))
 (segment (start 176.4675 99.4675) (end 177.71 100.71) (width 0.25) (layer "F.Cu") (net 2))
 (segment (start 167.894 99.06) (end 169.164 97.79) (width 0.25) (layer "F.Cu") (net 2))
 (segment (start 167.832 99.4675) (end 170.942 99.4675) (width 0.25) (layer "F.Cu") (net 2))
 (segment (start 159.0315 100.71) (end 159.4115 100.33) (width 0.25) (layer "F.Cu") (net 2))
 (segment (start 169.265 94.062) (end 168.35 94.977) (width 0.25) (layer "F.Cu") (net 2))
 (segment (start 162.56 101.6) (end 143.51 101.6) (width 0.25) (layer "F.Cu") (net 2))
 (segment (start 156.972 92.71) (end 157.988 93.726) (width 0.15) (layer "F.Cu") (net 2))
 (segment (start 169.42 89.918) (end 169.42 89.882) (width 0.25) (layer "F.Cu") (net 2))
 (segment (start 140.643 100.71) (end 141.8855 99.4675) (width 0.25) (layer "F.Cu") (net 2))
 (segment (start 169.164 96.012) (end 169.164 95.791) (width 0.25) (layer "F.Cu") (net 2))
 (segment (start 157.988 89.963) (end 158.069 89.882) (width 0.15) (layer "F.Cu") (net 2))
 (segment (start 102.4625 99.4675) (end 117.4125 99.4675) (width 0.25) (layer "F.Cu") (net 2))
 (via (at 169.164 96.012) (size 0.8) (drill 0.4) (layers "F.Cu" "B.Cu") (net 2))
 (via (at 193.04 94.488) (size 0.8) (drill 0.4) (layers "F.Cu" "B.Cu") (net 2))
 (via (at 169.164 97.79) (size 0.8) (drill 0.4) (layers "F.Cu" "B.Cu") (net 2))
 (via (at 162.56 97.028) (size 0.8) (drill 0.4) (layers "F.Cu" "B.Cu") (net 2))
 (via (at 165.862 99.06) (size 0.8) (drill 0.4) (layers "F.Cu" "B.Cu") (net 2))
 (segment (start 164.592 99.06) (end 165.862 99.06) (width 0.25) (layer "B.Cu") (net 2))
 (segment (start 193.04 94.488) (end 187.49 100.038) (width 0.25) (layer "B.Cu") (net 2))
 (segment (start 187.49 100.038) (end 187.49 103.21) (width 0.25) (layer "B.Cu") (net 2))
 (segment (start 162.56 97.028) (end 164.592 99.06) (width 0.25) (layer "B.Cu") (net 2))
 (segment (start 169.164 97.79) (end 169.164 96.012) (width 0.25) (layer "B.Cu") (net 2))
 (segment (start 170.688 100.838) (end 172.682 100.838) (width 0.25) (layer "F.Cu") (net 13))
 (segment (start 159.638 97.41) (end 159.766 97.282) (width 0.25) (layer "F.Cu") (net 13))
 (segment (start 158.025 97.41) (end 159.638 97.41) (width 0.25) (layer "F.Cu") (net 13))
 (segment (start 172.682 100.838) (end 172.81 100.71) (width 0.25) (layer "F.Cu") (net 13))
 (via (at 159.766 97.282) (size 0.8) (drill 0.4) (layers "F.Cu" "B.Cu") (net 13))
 (via (at 170.688 100.838) (size 0.8) (drill 0.4) (layers "F.Cu" "B.Cu") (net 13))
 (segment (start 161.544 97.282) (end 164.084 99.822) (width 0.25) (layer "B.Cu") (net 13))
 (segment (start 169.672 99.822) (end 170.688 100.838) (width 0.25) (layer "B.Cu") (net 13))
 (segment (start 164.084 99.822) (end 169.672 99.822) (width 0.25) (layer "B.Cu") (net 13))
 (segment (start 159.766 97.282) (end 161.544 97.282) (width 0.25) (layer "B.Cu") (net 13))
 (segment (start 178.308 105.918) (end 177.6965 105.918) (width 0.25) (layer "F.Cu") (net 14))
 (segment (start 177.71 97.41) (end 179.324 99.024) (width 0.25) (layer "F.Cu") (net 14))
 (segment (start 179.324 104.902) (end 178.308 105.918) (width 0.25) (layer "F.Cu") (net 14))
 (segment (start 179.324 99.024) (end 179.324 104.902) (width 0.25) (layer "F.Cu") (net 14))
 (segment (start 151.13 100.838) (end 152.997 100.838) (width 0.25) (layer "F.Cu") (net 11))
 (segment (start 152.997 100.838) (end 153.125 100.71) (width 0.25) (layer "F.Cu") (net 11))
 (segment (start 140.08 97.41) (end 140.208 97.282) (width 0.25) (layer "F.Cu") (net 11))
 (segment (start 138.34 97.41) (end 140.08 97.41) (width 0.25) (layer "F.Cu") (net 11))
 (via (at 140.208 97.282) (size 0.8) (drill 0.4) (layers "F.Cu" "B.Cu") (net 11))
 (via (at 151.13 100.838) (size 0.8) (drill 0.4) (layers "F.Cu" "B.Cu") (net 11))
 (segment (start 140.208 97.282) (end 143.764 100.838) (width 0.25) (layer "B.Cu") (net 11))
 (segment (start 143.764 100.838) (end 151.13 100.838) (width 0.25) (layer "B.Cu") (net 11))
 (segment (start 118.655 97.41) (end 120.522 97.41) (width 0.25) (layer "F.Cu") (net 4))
 (segment (start 131.572 100.584) (end 133.314 100.584) (width 0.25) (layer "F.Cu") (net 4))
 (segment (start 133.314 100.584) (end 133.44 100.71) (width 0.25) (layer "F.Cu") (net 4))
 (segment (start 120.522 97.41) (end 120.65 97.282) (width 0.25) (layer "F.Cu") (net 4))
 (via (at 131.572 100.584) (size 0.8) (drill 0.4) (layers "F.Cu" "B.Cu") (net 4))
 (via (at 120.65 97.282) (size 0.8) (drill 0.4) (layers "F.Cu" "B.Cu") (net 4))
 (segment (start 120.65 97.282) (end 123.952 100.584) (width 0.25) (layer "B.Cu") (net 4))
 (segment (start 123.952 100.584) (end 131.572 100.584) (width 0.25) (layer "B.Cu") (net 4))
 (segment (start 100.71 97.41) (end 100.838 97.282) (width 0.25) (layer "F.Cu") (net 3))
 (segment (start 113.627 100.838) (end 113.755 100.71) (width 0.25) (layer "F.Cu") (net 3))
 (segment (start 98.97 97.41) (end 100.71 97.41) (width 0.25) (layer "F.Cu") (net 3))
 (segment (start 112.014 100.838) (end 113.627 100.838) (width 0.25) (layer "F.Cu") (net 3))
 (via (at 112.014 100.838) (size 0.8) (drill 0.4) (layers "F.Cu" "B.Cu") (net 3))
 (via (at 100.838 97.282) (size 0.8) (drill 0.4) (layers "F.Cu" "B.Cu") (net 3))
 (segment (start 100.838 97.282) (end 104.394 100.838) (width 0.25) (layer "B.Cu") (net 3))
 (segment (start 104.394 100.838) (end 112.014 100.838) (width 0.25) (layer "B.Cu") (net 3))
 (segment (start 157.988 88.138) (end 161.117 88.138) (width 0.15) (layer "F.Cu") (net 12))
 (segment (start 161.117 88.138) (end 166.35 93.371) (width 0.15) (layer "F.Cu") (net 12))
 (segment (start 166.35 93.371) (end 166.35 94.977) (width 0.15) (layer "F.Cu") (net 12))
 (segment (start 157.988 91.901) (end 161.498241 91.901) (width 0.15) (layer "F.Cu") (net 18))
 (segment (start 161.498241 91.901) (end 163.35 93.752759) (width 0.15) (layer "F.Cu") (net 18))
 (segment (start 163.35 93.752759) (end 163.35 94.977) (width 0.15) (layer "F.Cu") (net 18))
 (segment (start 155.956 103.378) (end 151.892 103.378) (width 0.25) (layer "F.Cu") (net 9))
 (segment (start 164.084 105.918) (end 166.878 105.918) (width 0.25) (layer "F.Cu") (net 9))
 (segment (start 162.466 105.791) (end 158.369 105.791) (width 0.25) (layer "F.Cu") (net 9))
 (segment (start 158.369 105.791) (end 155.956 103.378) (width 0.25) (layer "F.Cu") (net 9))
 (segment (start 164.084 105.918) (end 162.593 105.918) (width 0.25) (layer "F.Cu") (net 9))
 (segment (start 175.8715 105.918) (end 174.498 105.918) (width 0.25) (layer "F.Cu") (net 9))
 (segment (start 174.498 105.918) (end 172.466 105.918) (width 0.25) (layer "F.Cu") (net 9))
 (segment (start 162.593 105.918) (end 162.466 105.791) (width 0.25) (layer "F.Cu") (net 9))
 (via (at 166.878 105.918) (size 0.8) (drill 0.4) (layers "F.Cu" "B.Cu") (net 9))
 (via (at 172.466 105.918) (size 0.8) (drill 0.4) (layers "F.Cu" "B.Cu") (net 9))
 (segment (start 166.878 105.918) (end 172.466 105.918) (width 0.25) (layer "B.Cu") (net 9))
 (segment (start 153.289 107.061) (end 153.035 107.061) (width 0.25) (layer "F.Cu") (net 10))
 (segment (start 153.035 107.061) (end 149.352 103.378) (width 0.25) (layer "F.Cu") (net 10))
 (segment (start 162.466 107.061) (end 153.289 107.061) (width 0.25) (layer "F.Cu") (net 10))
 (segment (start 183.7925 103.378) (end 185.8245 101.346) (width 0.25) (layer "F.Cu") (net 5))
 (segment (start 165.989 108.331) (end 162.466 108.331) (width 0.25) (layer "F.Cu") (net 5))
 (segment (start 197.826 101.346) (end 198.99 102.51) (width 0.25) (layer "F.Cu") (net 5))
 (segment (start 162.466 108.331) (end 152.273 108.331) (width 0.25) (layer "F.Cu") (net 5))
 (segment (start 175.9185 111.252) (end 168.91 111.252) (width 0.25) (layer "F.Cu") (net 5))
 (segment (start 168.91 111.252) (end 165.989 108.331) (width 0.25) (layer "F.Cu") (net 5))
 (segment (start 151.765 108.331) (end 146.812 103.378) (width 0.25) (layer "F.Cu") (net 5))
 (segment (start 185.8245 101.346) (end 197.826 101.346) (width 0.25) (layer "F.Cu") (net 5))
 (segment (start 152.273 108.331) (end 151.765 108.331) (width 0.25) (layer "F.Cu") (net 5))
 (segment (start 183.7925 103.378) (end 175.9185 111.252) (width 0.25) (layer "F.Cu") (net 5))
 (segment (start 165.862 102.108) (end 145.542 102.108) (width 0.25) (layer "F.Cu") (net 6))
 (segment (start 167.894 104.14) (end 165.862 102.108) (width 0.25) (layer "F.Cu") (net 6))
 (segment (start 169.766 109.601) (end 169.037 109.601) (width 0.25) (layer "F.Cu") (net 6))
 (segment (start 169.037 109.601) (end 167.894 108.458) (width 0.25) (layer "F.Cu") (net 6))
 (segment (start 145.542 102.108) (end 144.272 103.378) (width 0.25) (layer "F.Cu") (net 6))
 (segment (start 167.894 108.458) (end 167.894 104.14) (width 0.25) (layer "F.Cu") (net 6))
 (segment (start 182.88 96.52) (end 182.88 95.6545) (width 0.25) (layer "F.Cu") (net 7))
 (segment (start 183.9605 94.91) (end 187.49 94.91) (width 0.25) (layer "F.Cu") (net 7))
 (segment (start 183.7925 94.742) (end 183.9605 94.91) (width 0.25) (layer "F.Cu") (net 7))
 (segment (start 183.896 97.536) (end 182.88 96.52) (width 0.25) (layer "F.Cu") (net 7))
 (segment (start 173.609 108.331) (end 174.244 107.696) (width 0.25) (layer "F.Cu") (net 7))
 (segment (start 182.88 95.6545) (end 183.7925 94.742) (width 0.25) (layer "F.Cu") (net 7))
 (segment (start 169.766 108.331) (end 173.609 108.331) (width 0.25) (layer "F.Cu") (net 7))
 (via (at 183.896 97.536) (size 0.8) (drill 0.4) (layers "F.Cu" "B.Cu") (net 7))
 (via (at 174.244 107.696) (size 0.8) (drill 0.4) (layers "F.Cu" "B.Cu") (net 7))
 (segment (start 178.562 103.378) (end 181.864 103.378) (width 0.25) (layer "B.Cu") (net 7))
 (segment (start 181.864 103.378) (end 183.896 101.346) (width 0.25) (layer "B.Cu") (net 7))
 (segment (start 174.244 107.696) (end 178.562 103.378) (width 0.25) (layer "B.Cu") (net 7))
 (segment (start 183.896 101.346) (end 183.896 97.536) (width 0.25) (layer "B.Cu") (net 7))
 (segment (start 173.101 107.061) (end 173.482 106.68) (width 0.25) (layer "F.Cu") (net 8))
 (segment (start 183.7925 99.06) (end 194.44 99.06) (width 0.25) (layer "F.Cu") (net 8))
 (segment (start 182.88 99.9725) (end 183.7925 99.06) (width 0.25) (layer "F.Cu") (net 8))
 (segment (start 169.766 107.061) (end 173.101 107.061) (width 0.25) (layer "F.Cu") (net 8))
 (segment (start 182.88 100.584) (end 182.88 99.9725) (width 0.25) (layer "F.Cu") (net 8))
 (segment (start 194.44 99.06) (end 198.59 94.91) (width 0.25) (layer "F.Cu") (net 8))
 (via (at 182.88 100.584) (size 0.8) (drill 0.4) (layers "F.Cu" "B.Cu") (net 8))
 (via (at 173.482 106.68) (size 0.8) (drill 0.4) (layers "F.Cu" "B.Cu") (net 8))
 (segment (start 177.8 102.362) (end 180.34 102.362) (width 0.25) (layer "B.Cu") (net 8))
 (segment (start 181.102 102.362) (end 182.88 100.584) (width 0.25) (layer "B.Cu") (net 8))
 (segment (start 173.482 106.68) (end 177.8 102.362) (width 0.25) (layer "B.Cu") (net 8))
 (segment (start 180.34 102.362) (end 180.594 102.362) (width 0.25) (layer "B.Cu") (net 8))
 (segment (start 180.594 102.362) (end 181.102 102.362) (width 0.25) (layer "B.Cu") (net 8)))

